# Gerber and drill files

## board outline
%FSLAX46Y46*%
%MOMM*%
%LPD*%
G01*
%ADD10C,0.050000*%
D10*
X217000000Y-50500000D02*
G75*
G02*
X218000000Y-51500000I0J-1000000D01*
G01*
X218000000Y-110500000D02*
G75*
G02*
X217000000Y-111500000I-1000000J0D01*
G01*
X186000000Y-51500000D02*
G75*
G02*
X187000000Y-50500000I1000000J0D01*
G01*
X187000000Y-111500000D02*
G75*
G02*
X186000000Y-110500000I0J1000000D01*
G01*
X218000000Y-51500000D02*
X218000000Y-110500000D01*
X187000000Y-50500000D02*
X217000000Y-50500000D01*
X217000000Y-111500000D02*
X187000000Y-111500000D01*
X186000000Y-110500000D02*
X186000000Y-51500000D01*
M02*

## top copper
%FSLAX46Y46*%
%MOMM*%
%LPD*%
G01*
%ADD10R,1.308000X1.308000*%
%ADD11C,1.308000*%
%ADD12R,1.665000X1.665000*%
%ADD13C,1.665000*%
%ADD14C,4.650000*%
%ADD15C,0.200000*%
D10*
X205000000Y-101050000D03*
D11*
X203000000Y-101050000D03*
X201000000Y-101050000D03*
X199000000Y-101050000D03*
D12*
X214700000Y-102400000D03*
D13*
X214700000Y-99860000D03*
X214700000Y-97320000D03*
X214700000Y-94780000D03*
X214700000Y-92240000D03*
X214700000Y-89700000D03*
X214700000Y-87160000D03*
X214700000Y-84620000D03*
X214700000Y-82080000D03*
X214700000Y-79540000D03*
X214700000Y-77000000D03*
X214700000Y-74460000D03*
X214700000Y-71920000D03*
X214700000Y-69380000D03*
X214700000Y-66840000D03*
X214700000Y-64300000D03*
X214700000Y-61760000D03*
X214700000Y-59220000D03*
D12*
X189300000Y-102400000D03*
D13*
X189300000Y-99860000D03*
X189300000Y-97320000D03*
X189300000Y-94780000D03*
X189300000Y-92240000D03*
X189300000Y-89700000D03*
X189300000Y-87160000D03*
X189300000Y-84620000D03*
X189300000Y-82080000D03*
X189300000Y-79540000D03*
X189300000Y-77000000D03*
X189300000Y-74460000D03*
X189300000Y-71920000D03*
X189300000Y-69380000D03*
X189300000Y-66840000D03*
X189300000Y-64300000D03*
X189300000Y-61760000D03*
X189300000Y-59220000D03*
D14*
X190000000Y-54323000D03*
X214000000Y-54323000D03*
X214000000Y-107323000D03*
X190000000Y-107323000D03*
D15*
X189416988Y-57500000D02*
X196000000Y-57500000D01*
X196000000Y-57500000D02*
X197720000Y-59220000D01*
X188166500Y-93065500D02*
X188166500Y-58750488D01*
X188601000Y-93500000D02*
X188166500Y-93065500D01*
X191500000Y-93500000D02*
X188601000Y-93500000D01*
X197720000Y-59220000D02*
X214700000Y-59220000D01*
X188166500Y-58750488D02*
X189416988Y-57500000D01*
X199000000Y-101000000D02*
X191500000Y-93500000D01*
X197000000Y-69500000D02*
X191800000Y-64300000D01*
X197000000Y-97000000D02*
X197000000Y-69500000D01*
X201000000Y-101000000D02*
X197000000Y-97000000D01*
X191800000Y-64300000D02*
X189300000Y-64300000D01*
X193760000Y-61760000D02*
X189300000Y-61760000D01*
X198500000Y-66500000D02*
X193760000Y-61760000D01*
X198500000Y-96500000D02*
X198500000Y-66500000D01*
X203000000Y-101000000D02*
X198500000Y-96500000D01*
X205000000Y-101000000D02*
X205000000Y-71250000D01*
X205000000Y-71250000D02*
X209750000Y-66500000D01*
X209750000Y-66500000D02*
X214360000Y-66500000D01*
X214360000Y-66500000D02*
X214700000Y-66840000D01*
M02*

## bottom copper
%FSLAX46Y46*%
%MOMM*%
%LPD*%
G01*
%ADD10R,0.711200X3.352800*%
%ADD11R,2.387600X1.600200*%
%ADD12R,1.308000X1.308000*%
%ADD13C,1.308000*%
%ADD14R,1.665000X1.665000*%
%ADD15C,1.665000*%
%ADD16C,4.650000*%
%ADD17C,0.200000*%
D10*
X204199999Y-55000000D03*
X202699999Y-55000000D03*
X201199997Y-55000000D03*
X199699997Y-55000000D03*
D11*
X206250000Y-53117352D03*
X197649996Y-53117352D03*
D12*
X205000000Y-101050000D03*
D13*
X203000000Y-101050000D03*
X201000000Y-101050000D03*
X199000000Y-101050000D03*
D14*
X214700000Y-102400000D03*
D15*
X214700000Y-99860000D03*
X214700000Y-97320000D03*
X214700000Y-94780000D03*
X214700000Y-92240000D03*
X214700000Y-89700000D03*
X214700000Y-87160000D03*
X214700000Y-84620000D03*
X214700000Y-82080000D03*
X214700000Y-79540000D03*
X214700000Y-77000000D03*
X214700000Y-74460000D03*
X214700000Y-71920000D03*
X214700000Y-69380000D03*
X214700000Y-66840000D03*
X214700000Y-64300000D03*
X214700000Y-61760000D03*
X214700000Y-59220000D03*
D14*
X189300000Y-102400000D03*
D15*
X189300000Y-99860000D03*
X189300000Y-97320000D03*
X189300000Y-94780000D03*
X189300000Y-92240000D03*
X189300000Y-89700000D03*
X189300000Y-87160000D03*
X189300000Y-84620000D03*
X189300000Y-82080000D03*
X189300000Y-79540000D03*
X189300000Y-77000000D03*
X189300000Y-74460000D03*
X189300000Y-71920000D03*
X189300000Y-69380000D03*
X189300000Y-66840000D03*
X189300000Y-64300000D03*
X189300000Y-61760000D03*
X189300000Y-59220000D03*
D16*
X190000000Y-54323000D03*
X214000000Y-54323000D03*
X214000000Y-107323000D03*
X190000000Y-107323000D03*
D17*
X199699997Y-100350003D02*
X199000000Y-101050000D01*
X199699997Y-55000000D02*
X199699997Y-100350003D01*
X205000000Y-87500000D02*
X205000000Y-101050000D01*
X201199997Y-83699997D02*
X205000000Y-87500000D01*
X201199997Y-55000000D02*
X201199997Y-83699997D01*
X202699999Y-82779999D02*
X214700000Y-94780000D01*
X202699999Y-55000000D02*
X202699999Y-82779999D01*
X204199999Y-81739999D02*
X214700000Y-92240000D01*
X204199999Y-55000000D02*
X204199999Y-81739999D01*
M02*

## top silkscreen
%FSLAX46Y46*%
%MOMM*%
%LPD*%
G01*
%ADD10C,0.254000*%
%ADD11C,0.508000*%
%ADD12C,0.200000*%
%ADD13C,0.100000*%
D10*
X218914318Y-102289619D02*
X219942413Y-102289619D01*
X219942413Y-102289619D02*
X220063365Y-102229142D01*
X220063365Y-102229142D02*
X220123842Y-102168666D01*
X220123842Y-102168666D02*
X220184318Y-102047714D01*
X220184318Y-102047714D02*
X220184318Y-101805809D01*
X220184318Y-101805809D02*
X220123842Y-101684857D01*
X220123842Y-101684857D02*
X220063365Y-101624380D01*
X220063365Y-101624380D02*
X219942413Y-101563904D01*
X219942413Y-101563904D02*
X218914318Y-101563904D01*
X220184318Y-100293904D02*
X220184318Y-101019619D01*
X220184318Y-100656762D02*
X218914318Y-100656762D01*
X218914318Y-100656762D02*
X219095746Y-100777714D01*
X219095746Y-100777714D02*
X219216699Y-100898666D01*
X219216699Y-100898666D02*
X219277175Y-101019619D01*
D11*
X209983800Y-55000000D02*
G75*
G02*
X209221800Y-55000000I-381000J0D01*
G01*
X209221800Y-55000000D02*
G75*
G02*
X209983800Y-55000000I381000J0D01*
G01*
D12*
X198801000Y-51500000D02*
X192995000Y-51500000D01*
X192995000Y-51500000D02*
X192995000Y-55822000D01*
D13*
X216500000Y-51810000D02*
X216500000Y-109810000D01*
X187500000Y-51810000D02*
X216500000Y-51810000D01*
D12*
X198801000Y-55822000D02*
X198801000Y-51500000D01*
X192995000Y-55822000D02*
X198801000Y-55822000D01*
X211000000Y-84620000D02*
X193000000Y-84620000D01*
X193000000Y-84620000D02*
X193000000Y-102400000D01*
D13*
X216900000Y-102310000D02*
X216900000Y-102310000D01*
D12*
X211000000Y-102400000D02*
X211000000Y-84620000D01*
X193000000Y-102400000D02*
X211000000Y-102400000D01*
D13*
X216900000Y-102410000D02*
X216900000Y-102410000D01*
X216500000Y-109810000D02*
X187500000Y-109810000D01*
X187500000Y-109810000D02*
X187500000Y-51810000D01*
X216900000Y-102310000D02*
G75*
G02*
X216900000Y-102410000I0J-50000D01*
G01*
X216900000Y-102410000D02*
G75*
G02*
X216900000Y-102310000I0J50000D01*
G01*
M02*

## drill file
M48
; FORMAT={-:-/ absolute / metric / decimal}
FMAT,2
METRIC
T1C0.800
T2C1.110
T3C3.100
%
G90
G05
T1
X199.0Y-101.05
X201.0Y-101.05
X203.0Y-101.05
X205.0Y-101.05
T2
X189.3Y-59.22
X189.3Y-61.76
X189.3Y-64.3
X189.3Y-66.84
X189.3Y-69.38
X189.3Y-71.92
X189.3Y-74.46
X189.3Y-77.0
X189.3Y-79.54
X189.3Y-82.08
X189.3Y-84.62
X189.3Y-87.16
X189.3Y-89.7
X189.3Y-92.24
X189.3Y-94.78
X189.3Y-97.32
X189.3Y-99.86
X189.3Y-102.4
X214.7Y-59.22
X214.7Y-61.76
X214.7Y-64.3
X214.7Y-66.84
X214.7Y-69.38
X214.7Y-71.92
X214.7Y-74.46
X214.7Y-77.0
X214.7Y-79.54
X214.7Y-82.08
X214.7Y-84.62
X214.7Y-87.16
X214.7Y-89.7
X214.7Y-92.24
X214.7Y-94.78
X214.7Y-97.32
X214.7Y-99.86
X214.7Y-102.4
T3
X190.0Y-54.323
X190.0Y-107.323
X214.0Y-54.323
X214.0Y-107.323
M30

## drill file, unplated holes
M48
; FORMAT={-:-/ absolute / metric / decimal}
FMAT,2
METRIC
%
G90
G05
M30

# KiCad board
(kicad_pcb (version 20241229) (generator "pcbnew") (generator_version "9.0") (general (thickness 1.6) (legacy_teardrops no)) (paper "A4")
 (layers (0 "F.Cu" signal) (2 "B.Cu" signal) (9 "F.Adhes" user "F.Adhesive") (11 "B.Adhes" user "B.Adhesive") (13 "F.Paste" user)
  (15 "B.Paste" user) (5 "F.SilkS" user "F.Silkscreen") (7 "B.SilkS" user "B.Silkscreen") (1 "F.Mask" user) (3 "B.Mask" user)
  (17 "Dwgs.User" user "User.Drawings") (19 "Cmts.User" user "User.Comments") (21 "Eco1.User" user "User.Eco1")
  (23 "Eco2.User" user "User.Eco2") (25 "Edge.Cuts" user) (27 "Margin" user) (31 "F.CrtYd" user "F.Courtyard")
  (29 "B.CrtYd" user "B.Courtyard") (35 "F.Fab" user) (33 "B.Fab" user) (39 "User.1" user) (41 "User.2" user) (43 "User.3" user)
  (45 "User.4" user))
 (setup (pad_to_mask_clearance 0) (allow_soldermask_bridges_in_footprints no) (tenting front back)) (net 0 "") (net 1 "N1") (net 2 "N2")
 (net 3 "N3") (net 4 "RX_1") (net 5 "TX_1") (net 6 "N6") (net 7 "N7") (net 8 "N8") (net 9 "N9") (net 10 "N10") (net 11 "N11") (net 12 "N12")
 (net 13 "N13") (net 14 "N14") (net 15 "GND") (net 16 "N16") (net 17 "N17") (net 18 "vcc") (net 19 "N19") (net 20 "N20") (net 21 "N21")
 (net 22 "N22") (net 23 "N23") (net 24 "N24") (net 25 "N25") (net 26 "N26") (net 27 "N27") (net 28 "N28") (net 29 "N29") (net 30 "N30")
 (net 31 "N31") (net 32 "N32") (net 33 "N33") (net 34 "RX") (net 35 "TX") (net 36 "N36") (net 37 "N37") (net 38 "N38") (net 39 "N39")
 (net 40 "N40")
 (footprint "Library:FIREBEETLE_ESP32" (layer "F.Cu") (at 202 77 -90)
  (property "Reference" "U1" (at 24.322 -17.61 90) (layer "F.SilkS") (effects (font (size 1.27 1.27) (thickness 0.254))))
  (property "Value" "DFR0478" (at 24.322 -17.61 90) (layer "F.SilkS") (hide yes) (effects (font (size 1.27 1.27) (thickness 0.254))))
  (fp_line (start -25.19 14.5) (end -25.19 -14.5) (stroke (width 0.1) (type solid)) (layer "F.SilkS"))
  (fp_line (start 32.81 14.5) (end -25.19 14.5) (stroke (width 0.1) (type solid)) (layer "F.SilkS"))
  (fp_line (start -25.5 9.005) (end -21.178 9.005) (stroke (width 0.2) (type solid)) (layer "F.SilkS"))
  (fp_line (start -21.178 9.005) (end -21.178 3.199) (stroke (width 0.2) (type solid)) (layer "F.SilkS"))
  (fp_line (start 7.62 9) (end 25.4 9) (stroke (width 0.2) (type solid)) (layer "F.SilkS"))
  (fp_line (start 25.4 9) (end 25.4 -9) (stroke (width 0.2) (type solid)) (layer "F.SilkS"))
  (fp_line (start -25.5 3.199) (end -25.5 9.005) (stroke (width 0.2) (type solid)) (layer "F.SilkS"))
  (fp_line (start -21.178 3.199) (end -25.5 3.199) (stroke (width 0.2) (type solid)) (layer "F.SilkS"))
  (fp_line (start 7.62 -9) (end 7.62 9) (stroke (width 0.2) (type solid)) (layer "F.SilkS"))
  (fp_line (start 25.4 -9) (end 7.62 -9) (stroke (width 0.2) (type solid)) (layer "F.SilkS"))
  (fp_line (start -25.19 -14.5) (end 32.81 -14.5) (stroke (width 0.1) (type solid)) (layer "F.SilkS"))
  (fp_line (start 32.81 -14.5) (end 32.81 14.5) (stroke (width 0.1) (type solid)) (layer "F.SilkS"))
  (fp_line (start 25.31 -14.9) (end 25.31 -14.9) (stroke (width 0.1) (type solid)) (layer "F.SilkS"))
  (fp_line (start 25.41 -14.9) (end 25.41 -14.9) (stroke (width 0.1) (type solid)) (layer "F.SilkS"))
  (fp_arc (start 25.31 -14.9) (mid 25.36 -14.95) (end 25.41 -14.9) (stroke (width 0.1) (type solid)) (layer "F.SilkS"))
  (fp_arc (start 25.41 -14.9) (mid 25.36 -14.85) (end 25.31 -14.9) (stroke (width 0.1) (type solid)) (layer "F.SilkS"))
  (pad "1" thru_hole rect (at 25.4 -12.7 270) (size 1.665 1.665) (drill 1.11) (layers "*.Cu" "*.Mask") (remove_unused_layers no)
   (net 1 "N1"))
  (pad "2" thru_hole circle (at 22.86 -12.7 270) (size 1.665 1.665) (drill 1.11) (layers "*.Cu" "*.Mask") (remove_unused_layers no)
   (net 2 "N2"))
  (pad "3" thru_hole circle (at 20.32 -12.7 270) (size 1.665 1.665) (drill 1.11) (layers "*.Cu" "*.Mask") (remove_unused_layers no)
   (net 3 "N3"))
  (pad "4" thru_hole circle (at 17.78 -12.7 270) (size 1.665 1.665) (drill 1.11) (layers "*.Cu" "*.Mask") (remove_unused_layers no)
   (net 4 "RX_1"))
  (pad "5" thru_hole circle (at 15.24 -12.7 270) (size 1.665 1.665) (drill 1.11) (layers "*.Cu" "*.Mask") (remove_unused_layers no)
   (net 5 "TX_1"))
  (pad "6" thru_hole circle (at 12.7 -12.7 270) (size 1.665 1.665) (drill 1.11) (layers "*.Cu" "*.Mask") (remove_unused_layers no)
   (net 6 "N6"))
  (pad "7" thru_hole circle (at 10.16 -12.7 270) (size 1.665 1.665) (drill 1.11) (layers "*.Cu" "*.Mask") (remove_unused_layers no)
   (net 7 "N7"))
  (pad "8" thru_hole circle (at 7.62 -12.7 270) (size 1.665 1.665) (drill 1.11) (layers "*.Cu" "*.Mask") (remove_unused_layers no)
   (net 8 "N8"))
  (pad "9" thru_hole circle (at 5.08 -12.7 270) (size 1.665 1.665) (drill 1.11) (layers "*.Cu" "*.Mask") (remove_unused_layers no)
   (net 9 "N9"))
  (pad "10" thru_hole circle (at 2.54 -12.7 270) (size 1.665 1.665) (drill 1.11) (layers "*.Cu" "*.Mask") (remove_unused_layers no)
   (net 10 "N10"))
  (pad "11" thru_hole circle (at 0 -12.7 270) (size 1.665 1.665) (drill 1.11) (layers "*.Cu" "*.Mask") (remove_unused_layers no)
   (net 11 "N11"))
  (pad "12" thru_hole circle (at -2.54 -12.7 270) (size 1.665 1.665) (drill 1.11) (layers "*.Cu" "*.Mask") (remove_unused_layers no)
   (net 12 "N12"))
  (pad "13" thru_hole circle (at -5.08 -12.7 270) (size 1.665 1.665) (drill 1.11) (layers "*.Cu" "*.Mask") (remove_unused_layers no)
   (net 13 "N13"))
  (pad "14" thru_hole circle (at -7.62 -12.7 270) (size 1.665 1.665) (drill 1.11) (layers "*.Cu" "*.Mask") (remove_unused_layers no)
   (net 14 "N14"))
  (pad "15" thru_hole circle (at -10.16 -12.7 270) (size 1.665 1.665) (drill 1.11) (layers "*.Cu" "*.Mask") (remove_unused_layers no)
   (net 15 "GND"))
  (pad "16" thru_hole circle (at -12.7 -12.7 270) (size 1.665 1.665) (drill 1.11) (layers "*.Cu" "*.Mask") (remove_unused_layers no)
   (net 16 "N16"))
  (pad "17" thru_hole circle (at -15.24 -12.7 270) (size 1.665 1.665) (drill 1.11) (layers "*.Cu" "*.Mask") (remove_unused_layers no)
   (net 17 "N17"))
  (pad "18" thru_hole circle (at -17.78 -12.7 270) (size 1.665 1.665) (drill 1.11) (layers "*.Cu" "*.Mask") (remove_unused_layers no)
   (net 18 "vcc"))
  (pad "19" thru_hole rect (at 25.4 12.7 270) (size 1.665 1.665) (drill 1.11) (layers "*.Cu" "*.Mask") (remove_unused_layers no)
   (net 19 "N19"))
  (pad "20" thru_hole circle (at 22.86 12.7 270) (size 1.665 1.665) (drill 1.11) (layers "*.Cu" "*.Mask") (remove_unused_layers no)
   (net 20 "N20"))
  (pad "21" thru_hole circle (at 20.32 12.7 270) (size 1.665 1.665) (drill 1.11) (layers "*.Cu" "*.Mask") (remove_unused_layers no)
   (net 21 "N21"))
  (pad "22" thru_hole circle (at 17.78 12.7 270) (size 1.665 1.665) (drill 1.11) (layers "*.Cu" "*.Mask") (remove_unused_layers no)
   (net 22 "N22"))
  (pad "23" thru_hole circle (at 15.24 12.7 270) (size 1.665 1.665) (drill 1.11) (layers "*.Cu" "*.Mask") (remove_unused_layers no)
   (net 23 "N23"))
  (pad "24" thru_hole circle (at 12.7 12.7 270) (size 1.665 1.665) (drill 1.11) (layers "*.Cu" "*.Mask") (remove_unused_layers no)
   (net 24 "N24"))
  (pad "25" thru_hole circle (at 10.16 12.7 270) (size 1.665 1.665) (drill 1.11) (layers "*.Cu" "*.Mask") (remove_unused_layers no)
   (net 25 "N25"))
  (pad "26" thru_hole circle (at 7.62 12.7 270) (size 1.665 1.665) (drill 1.11) (layers "*.Cu" "*.Mask") (remove_unused_layers no)
   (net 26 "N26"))
  (pad "27" thru_hole circle (at 5.08 12.7 270) (size 1.665 1.665) (drill 1.11) (layers "*.Cu" "*.Mask") (remove_unused_layers no)
   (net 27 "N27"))
  (pad "28" thru_hole circle (at 2.54 12.7 270) (size 1.665 1.665) (drill 1.11) (layers "*.Cu" "*.Mask") (remove_unused_layers no)
   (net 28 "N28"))
  (pad "29" thru_hole circle (at 0 12.7 270) (size 1.665 1.665) (drill 1.11) (layers "*.Cu" "*.Mask") (remove_unused_layers no)
   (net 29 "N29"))
  (pad "30" thru_hole circle (at -2.54 12.7 270) (size 1.665 1.665) (drill 1.11) (layers "*.Cu" "*.Mask") (remove_unused_layers no)
   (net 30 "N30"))
  (pad "31" thru_hole circle (at -5.08 12.7 270) (size 1.665 1.665) (drill 1.11) (layers "*.Cu" "*.Mask") (remove_unused_layers no)
   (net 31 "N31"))
  (pad "32" thru_hole circle (at -7.62 12.7 270) (size 1.665 1.665) (drill 1.11) (layers "*.Cu" "*.Mask") (remove_unused_layers no)
   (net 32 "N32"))
  (pad "33" thru_hole circle (at -10.16 12.7 270) (size 1.665 1.665) (drill 1.11) (layers "*.Cu" "*.Mask") (remove_unused_layers no)
   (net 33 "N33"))
  (pad "34" thru_hole circle (at -12.7 12.7 270) (size 1.665 1.665) (drill 1.11) (layers "*.Cu" "*.Mask") (remove_unused_layers no)
   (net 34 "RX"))
  (pad "35" thru_hole circle (at -15.24 12.7 270) (size 1.665 1.665) (drill 1.11) (layers "*.Cu" "*.Mask") (remove_unused_layers no)
   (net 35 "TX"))
  (pad "36" thru_hole circle (at -17.78 12.7 270) (size 1.665 1.665) (drill 1.11) (layers "*.Cu" "*.Mask") (remove_unused_layers no)
   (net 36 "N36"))
  (pad "MH1" thru_hole circle (at -22.677 12 270) (size 4.65 4.65) (drill 3.1) (layers "*.Cu" "*.Mask") (remove_unused_layers no)
   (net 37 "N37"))
  (pad "MH2" thru_hole circle (at -22.677 -12 270) (size 4.65 4.65) (drill 3.1) (layers "*.Cu" "*.Mask") (remove_unused_layers no)
   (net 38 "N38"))
  (pad "MH3" thru_hole circle (at 30.323 -12 270) (size 4.65 4.65) (drill 3.1) (layers "*.Cu" "*.Mask") (remove_unused_layers no)
   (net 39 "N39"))
  (pad "MH4" thru_hole circle (at 30.323 12 270) (size 4.65 4.65) (drill 3.1) (layers "*.Cu" "*.Mask") (remove_unused_layers no)
   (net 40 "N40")))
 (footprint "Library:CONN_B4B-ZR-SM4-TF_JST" (layer "B.Cu") (at 201.949998 53.1458 180)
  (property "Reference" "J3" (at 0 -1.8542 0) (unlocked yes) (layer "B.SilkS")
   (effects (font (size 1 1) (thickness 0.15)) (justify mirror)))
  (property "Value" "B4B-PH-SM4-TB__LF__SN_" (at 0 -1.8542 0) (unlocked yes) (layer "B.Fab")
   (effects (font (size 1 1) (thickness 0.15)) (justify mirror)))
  (fp_circle (center -7.652802 -1.8542) (end -7.271802 -1.8542) (stroke (width 0.508) (type solid)) (fill no) (layer "F.SilkS"))
  (pad "1" smd rect (at -2.250001 -1.8542 180) (size 0.7112 3.3528) (layers "B.Cu" "B.Mask" "B.Paste") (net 5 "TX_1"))
  (pad "2" smd rect (at -0.750001 -1.8542 180) (size 0.7112 3.3528) (layers "B.Cu" "B.Mask" "B.Paste") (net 4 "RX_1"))
  (pad "3" smd rect (at 0.750001 -1.8542 180) (size 0.7112 3.3528) (layers "B.Cu" "B.Mask" "B.Paste") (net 15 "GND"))
  (pad "4" smd rect (at 2.250001 -1.8542 180) (size 0.7112 3.3528) (layers "B.Cu" "B.Mask" "B.Paste") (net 18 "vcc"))
  (pad "5" smd rect (at -4.300002 0.028448 180) (size 2.3876 1.6002) (layers "B.Cu" "B.Mask" "B.Paste"))
  (pad "6" smd rect (at 4.300002 0.028448 180) (size 2.3876 1.6002) (layers "B.Cu" "B.Mask" "B.Paste")))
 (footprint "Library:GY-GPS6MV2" (layer "B.Cu") (at 202 84)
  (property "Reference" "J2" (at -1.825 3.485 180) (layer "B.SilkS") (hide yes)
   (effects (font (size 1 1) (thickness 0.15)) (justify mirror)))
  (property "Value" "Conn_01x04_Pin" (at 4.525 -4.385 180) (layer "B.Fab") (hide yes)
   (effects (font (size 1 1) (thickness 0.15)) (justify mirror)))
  (pad "1" thru_hole rect (at 3 17.05 180) (size 1.308 1.308) (drill 0.8) (layers "*.Cu" "*.Mask") (remove_unused_layers no) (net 15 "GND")
   (solder_mask_margin 0.102))
  (pad "2" thru_hole circle (at 1 17.05 180) (size 1.308 1.308) (drill 0.8) (layers "*.Cu" "*.Mask") (remove_unused_layers no) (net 35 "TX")
   (solder_mask_margin 0.102))
  (pad "3" thru_hole circle (at -1 17.05 180) (size 1.308 1.308) (drill 0.8) (layers "*.Cu" "*.Mask") (remove_unused_layers no)
   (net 34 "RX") (solder_mask_margin 0.102))
  (pad "4" thru_hole circle (at -3 17.05 180) (size 1.308 1.308) (drill 0.8) (layers "*.Cu" "*.Mask") (remove_unused_layers no)
   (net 18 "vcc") (solder_mask_margin 0.102)))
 (gr_line (start 186 110.5) (end 186 51.5) (stroke (width 0.05) (type default)) (layer "Edge.Cuts"))
 (gr_arc (start 218 110.5) (mid 217.707107 111.207107) (end 217 111.5) (stroke (width 0.05) (type default)) (layer "Edge.Cuts"))
 (gr_arc (start 187 111.5) (mid 186.292893 111.207107) (end 186 110.5) (stroke (width 0.05) (type default)) (layer "Edge.Cuts"))
 (gr_arc (start 186 51.5) (mid 186.292893 50.792893) (end 187 50.5) (stroke (width 0.05) (type default)) (layer "Edge.Cuts"))
 (gr_arc (start 217 50.5) (mid 217.707107 50.792893) (end 218 51.5) (stroke (width 0.05) (type default)) (layer "Edge.Cuts"))
 (gr_line (start 217 111.5) (end 187 111.5) (stroke (width 0.05) (type default)) (layer "Edge.Cuts"))
 (gr_line (start 187 50.5) (end 217 50.5) (stroke (width 0.05) (type default)) (layer "Edge.Cuts"))
 (gr_line (start 218 51.5) (end 218 110.5) (stroke (width 0.05) (type default)) (layer "Edge.Cuts"))
 (segment (start 205 101) (end 205 71.25) (width 0.2) (layer "F.Cu") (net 15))
 (segment (start 214.36 66.5) (end 214.7 66.84) (width 0.2) (layer "F.Cu") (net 15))
 (segment (start 205 71.25) (end 209.75 66.5) (width 0.2) (layer "F.Cu") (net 15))
 (segment (start 209.75 66.5) (end 214.36 66.5) (width 0.2) (layer "F.Cu") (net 15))
 (segment (start 201.199997 55) (end 201.199997 83.699997) (width 0.2) (layer "B.Cu") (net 15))
 (segment (start 205 87.5) (end 205 101.05) (width 0.2) (layer "B.Cu") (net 15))
 (segment (start 201.199997 83.699997) (end 205 87.5) (width 0.2) (layer "B.Cu") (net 15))
 (segment (start 198.5 96.5) (end 198.5 66.5) (width 0.2) (layer "F.Cu") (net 35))
 (segment (start 203 101) (end 198.5 96.5) (width 0.2) (layer "F.Cu") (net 35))
 (segment (start 193.76 61.76) (end 189.3 61.76) (width 0.2) (layer "F.Cu") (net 35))
 (segment (start 198.5 66.5) (end 193.76 61.76) (width 0.2) (layer "F.Cu") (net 35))
 (segment (start 201 101) (end 197 97) (width 0.2) (layer "F.Cu") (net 34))
 (segment (start 191.8 64.3) (end 189.3 64.3) (width 0.2) (layer "F.Cu") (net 34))
 (segment (start 197 69.5) (end 191.8 64.3) (width 0.2) (layer "F.Cu") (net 34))
 (segment (start 197 97) (end 197 69.5) (width 0.2) (layer "F.Cu") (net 34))
 (segment (start 199 101) (end 191.5 93.5) (width 0.2) (layer "F.Cu") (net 18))
 (segment (start 191.5 93.5) (end 188.601 93.5) (width 0.2) (layer "F.Cu") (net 18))
 (segment (start 197.72 59.22) (end 214.7 59.22) (width 0.2) (layer "F.Cu") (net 18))
 (segment (start 189.416988 57.5) (end 196 57.5) (width 0.2) (layer "F.Cu") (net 18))
 (segment (start 188.1665 58.750488) (end 189.416988 57.5) (width 0.2) (layer "F.Cu") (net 18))
 (segment (start 188.601 93.5) (end 188.1665 93.0655) (width 0.2) (layer "F.Cu") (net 18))
 (segment (start 196 57.5) (end 197.72 59.22) (width 0.2) (layer "F.Cu") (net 18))
 (segment (start 188.1665 93.0655) (end 188.1665 58.750488) (width 0.2) (layer "F.Cu") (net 18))
 (segment (start 199.699997 55) (end 199.699997 100.350003) (width 0.2) (layer "B.Cu") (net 18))
 (segment (start 199.699997 100.350003) (end 199 101.05) (width 0.2) (layer "B.Cu") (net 18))
 (segment (start 204.199999 55) (end 204.199999 81.739999) (width 0.2) (layer "B.Cu") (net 5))
 (segment (start 204.199999 81.739999) (end 214.7 92.24) (width 0.2) (layer "B.Cu") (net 5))
 (segment (start 202.699999 55) (end 202.699999 82.779999) (width 0.2) (layer "B.Cu") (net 4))
 (segment (start 202.699999 82.779999) (end 214.7 94.78) (width 0.2) (layer "B.Cu") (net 4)))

